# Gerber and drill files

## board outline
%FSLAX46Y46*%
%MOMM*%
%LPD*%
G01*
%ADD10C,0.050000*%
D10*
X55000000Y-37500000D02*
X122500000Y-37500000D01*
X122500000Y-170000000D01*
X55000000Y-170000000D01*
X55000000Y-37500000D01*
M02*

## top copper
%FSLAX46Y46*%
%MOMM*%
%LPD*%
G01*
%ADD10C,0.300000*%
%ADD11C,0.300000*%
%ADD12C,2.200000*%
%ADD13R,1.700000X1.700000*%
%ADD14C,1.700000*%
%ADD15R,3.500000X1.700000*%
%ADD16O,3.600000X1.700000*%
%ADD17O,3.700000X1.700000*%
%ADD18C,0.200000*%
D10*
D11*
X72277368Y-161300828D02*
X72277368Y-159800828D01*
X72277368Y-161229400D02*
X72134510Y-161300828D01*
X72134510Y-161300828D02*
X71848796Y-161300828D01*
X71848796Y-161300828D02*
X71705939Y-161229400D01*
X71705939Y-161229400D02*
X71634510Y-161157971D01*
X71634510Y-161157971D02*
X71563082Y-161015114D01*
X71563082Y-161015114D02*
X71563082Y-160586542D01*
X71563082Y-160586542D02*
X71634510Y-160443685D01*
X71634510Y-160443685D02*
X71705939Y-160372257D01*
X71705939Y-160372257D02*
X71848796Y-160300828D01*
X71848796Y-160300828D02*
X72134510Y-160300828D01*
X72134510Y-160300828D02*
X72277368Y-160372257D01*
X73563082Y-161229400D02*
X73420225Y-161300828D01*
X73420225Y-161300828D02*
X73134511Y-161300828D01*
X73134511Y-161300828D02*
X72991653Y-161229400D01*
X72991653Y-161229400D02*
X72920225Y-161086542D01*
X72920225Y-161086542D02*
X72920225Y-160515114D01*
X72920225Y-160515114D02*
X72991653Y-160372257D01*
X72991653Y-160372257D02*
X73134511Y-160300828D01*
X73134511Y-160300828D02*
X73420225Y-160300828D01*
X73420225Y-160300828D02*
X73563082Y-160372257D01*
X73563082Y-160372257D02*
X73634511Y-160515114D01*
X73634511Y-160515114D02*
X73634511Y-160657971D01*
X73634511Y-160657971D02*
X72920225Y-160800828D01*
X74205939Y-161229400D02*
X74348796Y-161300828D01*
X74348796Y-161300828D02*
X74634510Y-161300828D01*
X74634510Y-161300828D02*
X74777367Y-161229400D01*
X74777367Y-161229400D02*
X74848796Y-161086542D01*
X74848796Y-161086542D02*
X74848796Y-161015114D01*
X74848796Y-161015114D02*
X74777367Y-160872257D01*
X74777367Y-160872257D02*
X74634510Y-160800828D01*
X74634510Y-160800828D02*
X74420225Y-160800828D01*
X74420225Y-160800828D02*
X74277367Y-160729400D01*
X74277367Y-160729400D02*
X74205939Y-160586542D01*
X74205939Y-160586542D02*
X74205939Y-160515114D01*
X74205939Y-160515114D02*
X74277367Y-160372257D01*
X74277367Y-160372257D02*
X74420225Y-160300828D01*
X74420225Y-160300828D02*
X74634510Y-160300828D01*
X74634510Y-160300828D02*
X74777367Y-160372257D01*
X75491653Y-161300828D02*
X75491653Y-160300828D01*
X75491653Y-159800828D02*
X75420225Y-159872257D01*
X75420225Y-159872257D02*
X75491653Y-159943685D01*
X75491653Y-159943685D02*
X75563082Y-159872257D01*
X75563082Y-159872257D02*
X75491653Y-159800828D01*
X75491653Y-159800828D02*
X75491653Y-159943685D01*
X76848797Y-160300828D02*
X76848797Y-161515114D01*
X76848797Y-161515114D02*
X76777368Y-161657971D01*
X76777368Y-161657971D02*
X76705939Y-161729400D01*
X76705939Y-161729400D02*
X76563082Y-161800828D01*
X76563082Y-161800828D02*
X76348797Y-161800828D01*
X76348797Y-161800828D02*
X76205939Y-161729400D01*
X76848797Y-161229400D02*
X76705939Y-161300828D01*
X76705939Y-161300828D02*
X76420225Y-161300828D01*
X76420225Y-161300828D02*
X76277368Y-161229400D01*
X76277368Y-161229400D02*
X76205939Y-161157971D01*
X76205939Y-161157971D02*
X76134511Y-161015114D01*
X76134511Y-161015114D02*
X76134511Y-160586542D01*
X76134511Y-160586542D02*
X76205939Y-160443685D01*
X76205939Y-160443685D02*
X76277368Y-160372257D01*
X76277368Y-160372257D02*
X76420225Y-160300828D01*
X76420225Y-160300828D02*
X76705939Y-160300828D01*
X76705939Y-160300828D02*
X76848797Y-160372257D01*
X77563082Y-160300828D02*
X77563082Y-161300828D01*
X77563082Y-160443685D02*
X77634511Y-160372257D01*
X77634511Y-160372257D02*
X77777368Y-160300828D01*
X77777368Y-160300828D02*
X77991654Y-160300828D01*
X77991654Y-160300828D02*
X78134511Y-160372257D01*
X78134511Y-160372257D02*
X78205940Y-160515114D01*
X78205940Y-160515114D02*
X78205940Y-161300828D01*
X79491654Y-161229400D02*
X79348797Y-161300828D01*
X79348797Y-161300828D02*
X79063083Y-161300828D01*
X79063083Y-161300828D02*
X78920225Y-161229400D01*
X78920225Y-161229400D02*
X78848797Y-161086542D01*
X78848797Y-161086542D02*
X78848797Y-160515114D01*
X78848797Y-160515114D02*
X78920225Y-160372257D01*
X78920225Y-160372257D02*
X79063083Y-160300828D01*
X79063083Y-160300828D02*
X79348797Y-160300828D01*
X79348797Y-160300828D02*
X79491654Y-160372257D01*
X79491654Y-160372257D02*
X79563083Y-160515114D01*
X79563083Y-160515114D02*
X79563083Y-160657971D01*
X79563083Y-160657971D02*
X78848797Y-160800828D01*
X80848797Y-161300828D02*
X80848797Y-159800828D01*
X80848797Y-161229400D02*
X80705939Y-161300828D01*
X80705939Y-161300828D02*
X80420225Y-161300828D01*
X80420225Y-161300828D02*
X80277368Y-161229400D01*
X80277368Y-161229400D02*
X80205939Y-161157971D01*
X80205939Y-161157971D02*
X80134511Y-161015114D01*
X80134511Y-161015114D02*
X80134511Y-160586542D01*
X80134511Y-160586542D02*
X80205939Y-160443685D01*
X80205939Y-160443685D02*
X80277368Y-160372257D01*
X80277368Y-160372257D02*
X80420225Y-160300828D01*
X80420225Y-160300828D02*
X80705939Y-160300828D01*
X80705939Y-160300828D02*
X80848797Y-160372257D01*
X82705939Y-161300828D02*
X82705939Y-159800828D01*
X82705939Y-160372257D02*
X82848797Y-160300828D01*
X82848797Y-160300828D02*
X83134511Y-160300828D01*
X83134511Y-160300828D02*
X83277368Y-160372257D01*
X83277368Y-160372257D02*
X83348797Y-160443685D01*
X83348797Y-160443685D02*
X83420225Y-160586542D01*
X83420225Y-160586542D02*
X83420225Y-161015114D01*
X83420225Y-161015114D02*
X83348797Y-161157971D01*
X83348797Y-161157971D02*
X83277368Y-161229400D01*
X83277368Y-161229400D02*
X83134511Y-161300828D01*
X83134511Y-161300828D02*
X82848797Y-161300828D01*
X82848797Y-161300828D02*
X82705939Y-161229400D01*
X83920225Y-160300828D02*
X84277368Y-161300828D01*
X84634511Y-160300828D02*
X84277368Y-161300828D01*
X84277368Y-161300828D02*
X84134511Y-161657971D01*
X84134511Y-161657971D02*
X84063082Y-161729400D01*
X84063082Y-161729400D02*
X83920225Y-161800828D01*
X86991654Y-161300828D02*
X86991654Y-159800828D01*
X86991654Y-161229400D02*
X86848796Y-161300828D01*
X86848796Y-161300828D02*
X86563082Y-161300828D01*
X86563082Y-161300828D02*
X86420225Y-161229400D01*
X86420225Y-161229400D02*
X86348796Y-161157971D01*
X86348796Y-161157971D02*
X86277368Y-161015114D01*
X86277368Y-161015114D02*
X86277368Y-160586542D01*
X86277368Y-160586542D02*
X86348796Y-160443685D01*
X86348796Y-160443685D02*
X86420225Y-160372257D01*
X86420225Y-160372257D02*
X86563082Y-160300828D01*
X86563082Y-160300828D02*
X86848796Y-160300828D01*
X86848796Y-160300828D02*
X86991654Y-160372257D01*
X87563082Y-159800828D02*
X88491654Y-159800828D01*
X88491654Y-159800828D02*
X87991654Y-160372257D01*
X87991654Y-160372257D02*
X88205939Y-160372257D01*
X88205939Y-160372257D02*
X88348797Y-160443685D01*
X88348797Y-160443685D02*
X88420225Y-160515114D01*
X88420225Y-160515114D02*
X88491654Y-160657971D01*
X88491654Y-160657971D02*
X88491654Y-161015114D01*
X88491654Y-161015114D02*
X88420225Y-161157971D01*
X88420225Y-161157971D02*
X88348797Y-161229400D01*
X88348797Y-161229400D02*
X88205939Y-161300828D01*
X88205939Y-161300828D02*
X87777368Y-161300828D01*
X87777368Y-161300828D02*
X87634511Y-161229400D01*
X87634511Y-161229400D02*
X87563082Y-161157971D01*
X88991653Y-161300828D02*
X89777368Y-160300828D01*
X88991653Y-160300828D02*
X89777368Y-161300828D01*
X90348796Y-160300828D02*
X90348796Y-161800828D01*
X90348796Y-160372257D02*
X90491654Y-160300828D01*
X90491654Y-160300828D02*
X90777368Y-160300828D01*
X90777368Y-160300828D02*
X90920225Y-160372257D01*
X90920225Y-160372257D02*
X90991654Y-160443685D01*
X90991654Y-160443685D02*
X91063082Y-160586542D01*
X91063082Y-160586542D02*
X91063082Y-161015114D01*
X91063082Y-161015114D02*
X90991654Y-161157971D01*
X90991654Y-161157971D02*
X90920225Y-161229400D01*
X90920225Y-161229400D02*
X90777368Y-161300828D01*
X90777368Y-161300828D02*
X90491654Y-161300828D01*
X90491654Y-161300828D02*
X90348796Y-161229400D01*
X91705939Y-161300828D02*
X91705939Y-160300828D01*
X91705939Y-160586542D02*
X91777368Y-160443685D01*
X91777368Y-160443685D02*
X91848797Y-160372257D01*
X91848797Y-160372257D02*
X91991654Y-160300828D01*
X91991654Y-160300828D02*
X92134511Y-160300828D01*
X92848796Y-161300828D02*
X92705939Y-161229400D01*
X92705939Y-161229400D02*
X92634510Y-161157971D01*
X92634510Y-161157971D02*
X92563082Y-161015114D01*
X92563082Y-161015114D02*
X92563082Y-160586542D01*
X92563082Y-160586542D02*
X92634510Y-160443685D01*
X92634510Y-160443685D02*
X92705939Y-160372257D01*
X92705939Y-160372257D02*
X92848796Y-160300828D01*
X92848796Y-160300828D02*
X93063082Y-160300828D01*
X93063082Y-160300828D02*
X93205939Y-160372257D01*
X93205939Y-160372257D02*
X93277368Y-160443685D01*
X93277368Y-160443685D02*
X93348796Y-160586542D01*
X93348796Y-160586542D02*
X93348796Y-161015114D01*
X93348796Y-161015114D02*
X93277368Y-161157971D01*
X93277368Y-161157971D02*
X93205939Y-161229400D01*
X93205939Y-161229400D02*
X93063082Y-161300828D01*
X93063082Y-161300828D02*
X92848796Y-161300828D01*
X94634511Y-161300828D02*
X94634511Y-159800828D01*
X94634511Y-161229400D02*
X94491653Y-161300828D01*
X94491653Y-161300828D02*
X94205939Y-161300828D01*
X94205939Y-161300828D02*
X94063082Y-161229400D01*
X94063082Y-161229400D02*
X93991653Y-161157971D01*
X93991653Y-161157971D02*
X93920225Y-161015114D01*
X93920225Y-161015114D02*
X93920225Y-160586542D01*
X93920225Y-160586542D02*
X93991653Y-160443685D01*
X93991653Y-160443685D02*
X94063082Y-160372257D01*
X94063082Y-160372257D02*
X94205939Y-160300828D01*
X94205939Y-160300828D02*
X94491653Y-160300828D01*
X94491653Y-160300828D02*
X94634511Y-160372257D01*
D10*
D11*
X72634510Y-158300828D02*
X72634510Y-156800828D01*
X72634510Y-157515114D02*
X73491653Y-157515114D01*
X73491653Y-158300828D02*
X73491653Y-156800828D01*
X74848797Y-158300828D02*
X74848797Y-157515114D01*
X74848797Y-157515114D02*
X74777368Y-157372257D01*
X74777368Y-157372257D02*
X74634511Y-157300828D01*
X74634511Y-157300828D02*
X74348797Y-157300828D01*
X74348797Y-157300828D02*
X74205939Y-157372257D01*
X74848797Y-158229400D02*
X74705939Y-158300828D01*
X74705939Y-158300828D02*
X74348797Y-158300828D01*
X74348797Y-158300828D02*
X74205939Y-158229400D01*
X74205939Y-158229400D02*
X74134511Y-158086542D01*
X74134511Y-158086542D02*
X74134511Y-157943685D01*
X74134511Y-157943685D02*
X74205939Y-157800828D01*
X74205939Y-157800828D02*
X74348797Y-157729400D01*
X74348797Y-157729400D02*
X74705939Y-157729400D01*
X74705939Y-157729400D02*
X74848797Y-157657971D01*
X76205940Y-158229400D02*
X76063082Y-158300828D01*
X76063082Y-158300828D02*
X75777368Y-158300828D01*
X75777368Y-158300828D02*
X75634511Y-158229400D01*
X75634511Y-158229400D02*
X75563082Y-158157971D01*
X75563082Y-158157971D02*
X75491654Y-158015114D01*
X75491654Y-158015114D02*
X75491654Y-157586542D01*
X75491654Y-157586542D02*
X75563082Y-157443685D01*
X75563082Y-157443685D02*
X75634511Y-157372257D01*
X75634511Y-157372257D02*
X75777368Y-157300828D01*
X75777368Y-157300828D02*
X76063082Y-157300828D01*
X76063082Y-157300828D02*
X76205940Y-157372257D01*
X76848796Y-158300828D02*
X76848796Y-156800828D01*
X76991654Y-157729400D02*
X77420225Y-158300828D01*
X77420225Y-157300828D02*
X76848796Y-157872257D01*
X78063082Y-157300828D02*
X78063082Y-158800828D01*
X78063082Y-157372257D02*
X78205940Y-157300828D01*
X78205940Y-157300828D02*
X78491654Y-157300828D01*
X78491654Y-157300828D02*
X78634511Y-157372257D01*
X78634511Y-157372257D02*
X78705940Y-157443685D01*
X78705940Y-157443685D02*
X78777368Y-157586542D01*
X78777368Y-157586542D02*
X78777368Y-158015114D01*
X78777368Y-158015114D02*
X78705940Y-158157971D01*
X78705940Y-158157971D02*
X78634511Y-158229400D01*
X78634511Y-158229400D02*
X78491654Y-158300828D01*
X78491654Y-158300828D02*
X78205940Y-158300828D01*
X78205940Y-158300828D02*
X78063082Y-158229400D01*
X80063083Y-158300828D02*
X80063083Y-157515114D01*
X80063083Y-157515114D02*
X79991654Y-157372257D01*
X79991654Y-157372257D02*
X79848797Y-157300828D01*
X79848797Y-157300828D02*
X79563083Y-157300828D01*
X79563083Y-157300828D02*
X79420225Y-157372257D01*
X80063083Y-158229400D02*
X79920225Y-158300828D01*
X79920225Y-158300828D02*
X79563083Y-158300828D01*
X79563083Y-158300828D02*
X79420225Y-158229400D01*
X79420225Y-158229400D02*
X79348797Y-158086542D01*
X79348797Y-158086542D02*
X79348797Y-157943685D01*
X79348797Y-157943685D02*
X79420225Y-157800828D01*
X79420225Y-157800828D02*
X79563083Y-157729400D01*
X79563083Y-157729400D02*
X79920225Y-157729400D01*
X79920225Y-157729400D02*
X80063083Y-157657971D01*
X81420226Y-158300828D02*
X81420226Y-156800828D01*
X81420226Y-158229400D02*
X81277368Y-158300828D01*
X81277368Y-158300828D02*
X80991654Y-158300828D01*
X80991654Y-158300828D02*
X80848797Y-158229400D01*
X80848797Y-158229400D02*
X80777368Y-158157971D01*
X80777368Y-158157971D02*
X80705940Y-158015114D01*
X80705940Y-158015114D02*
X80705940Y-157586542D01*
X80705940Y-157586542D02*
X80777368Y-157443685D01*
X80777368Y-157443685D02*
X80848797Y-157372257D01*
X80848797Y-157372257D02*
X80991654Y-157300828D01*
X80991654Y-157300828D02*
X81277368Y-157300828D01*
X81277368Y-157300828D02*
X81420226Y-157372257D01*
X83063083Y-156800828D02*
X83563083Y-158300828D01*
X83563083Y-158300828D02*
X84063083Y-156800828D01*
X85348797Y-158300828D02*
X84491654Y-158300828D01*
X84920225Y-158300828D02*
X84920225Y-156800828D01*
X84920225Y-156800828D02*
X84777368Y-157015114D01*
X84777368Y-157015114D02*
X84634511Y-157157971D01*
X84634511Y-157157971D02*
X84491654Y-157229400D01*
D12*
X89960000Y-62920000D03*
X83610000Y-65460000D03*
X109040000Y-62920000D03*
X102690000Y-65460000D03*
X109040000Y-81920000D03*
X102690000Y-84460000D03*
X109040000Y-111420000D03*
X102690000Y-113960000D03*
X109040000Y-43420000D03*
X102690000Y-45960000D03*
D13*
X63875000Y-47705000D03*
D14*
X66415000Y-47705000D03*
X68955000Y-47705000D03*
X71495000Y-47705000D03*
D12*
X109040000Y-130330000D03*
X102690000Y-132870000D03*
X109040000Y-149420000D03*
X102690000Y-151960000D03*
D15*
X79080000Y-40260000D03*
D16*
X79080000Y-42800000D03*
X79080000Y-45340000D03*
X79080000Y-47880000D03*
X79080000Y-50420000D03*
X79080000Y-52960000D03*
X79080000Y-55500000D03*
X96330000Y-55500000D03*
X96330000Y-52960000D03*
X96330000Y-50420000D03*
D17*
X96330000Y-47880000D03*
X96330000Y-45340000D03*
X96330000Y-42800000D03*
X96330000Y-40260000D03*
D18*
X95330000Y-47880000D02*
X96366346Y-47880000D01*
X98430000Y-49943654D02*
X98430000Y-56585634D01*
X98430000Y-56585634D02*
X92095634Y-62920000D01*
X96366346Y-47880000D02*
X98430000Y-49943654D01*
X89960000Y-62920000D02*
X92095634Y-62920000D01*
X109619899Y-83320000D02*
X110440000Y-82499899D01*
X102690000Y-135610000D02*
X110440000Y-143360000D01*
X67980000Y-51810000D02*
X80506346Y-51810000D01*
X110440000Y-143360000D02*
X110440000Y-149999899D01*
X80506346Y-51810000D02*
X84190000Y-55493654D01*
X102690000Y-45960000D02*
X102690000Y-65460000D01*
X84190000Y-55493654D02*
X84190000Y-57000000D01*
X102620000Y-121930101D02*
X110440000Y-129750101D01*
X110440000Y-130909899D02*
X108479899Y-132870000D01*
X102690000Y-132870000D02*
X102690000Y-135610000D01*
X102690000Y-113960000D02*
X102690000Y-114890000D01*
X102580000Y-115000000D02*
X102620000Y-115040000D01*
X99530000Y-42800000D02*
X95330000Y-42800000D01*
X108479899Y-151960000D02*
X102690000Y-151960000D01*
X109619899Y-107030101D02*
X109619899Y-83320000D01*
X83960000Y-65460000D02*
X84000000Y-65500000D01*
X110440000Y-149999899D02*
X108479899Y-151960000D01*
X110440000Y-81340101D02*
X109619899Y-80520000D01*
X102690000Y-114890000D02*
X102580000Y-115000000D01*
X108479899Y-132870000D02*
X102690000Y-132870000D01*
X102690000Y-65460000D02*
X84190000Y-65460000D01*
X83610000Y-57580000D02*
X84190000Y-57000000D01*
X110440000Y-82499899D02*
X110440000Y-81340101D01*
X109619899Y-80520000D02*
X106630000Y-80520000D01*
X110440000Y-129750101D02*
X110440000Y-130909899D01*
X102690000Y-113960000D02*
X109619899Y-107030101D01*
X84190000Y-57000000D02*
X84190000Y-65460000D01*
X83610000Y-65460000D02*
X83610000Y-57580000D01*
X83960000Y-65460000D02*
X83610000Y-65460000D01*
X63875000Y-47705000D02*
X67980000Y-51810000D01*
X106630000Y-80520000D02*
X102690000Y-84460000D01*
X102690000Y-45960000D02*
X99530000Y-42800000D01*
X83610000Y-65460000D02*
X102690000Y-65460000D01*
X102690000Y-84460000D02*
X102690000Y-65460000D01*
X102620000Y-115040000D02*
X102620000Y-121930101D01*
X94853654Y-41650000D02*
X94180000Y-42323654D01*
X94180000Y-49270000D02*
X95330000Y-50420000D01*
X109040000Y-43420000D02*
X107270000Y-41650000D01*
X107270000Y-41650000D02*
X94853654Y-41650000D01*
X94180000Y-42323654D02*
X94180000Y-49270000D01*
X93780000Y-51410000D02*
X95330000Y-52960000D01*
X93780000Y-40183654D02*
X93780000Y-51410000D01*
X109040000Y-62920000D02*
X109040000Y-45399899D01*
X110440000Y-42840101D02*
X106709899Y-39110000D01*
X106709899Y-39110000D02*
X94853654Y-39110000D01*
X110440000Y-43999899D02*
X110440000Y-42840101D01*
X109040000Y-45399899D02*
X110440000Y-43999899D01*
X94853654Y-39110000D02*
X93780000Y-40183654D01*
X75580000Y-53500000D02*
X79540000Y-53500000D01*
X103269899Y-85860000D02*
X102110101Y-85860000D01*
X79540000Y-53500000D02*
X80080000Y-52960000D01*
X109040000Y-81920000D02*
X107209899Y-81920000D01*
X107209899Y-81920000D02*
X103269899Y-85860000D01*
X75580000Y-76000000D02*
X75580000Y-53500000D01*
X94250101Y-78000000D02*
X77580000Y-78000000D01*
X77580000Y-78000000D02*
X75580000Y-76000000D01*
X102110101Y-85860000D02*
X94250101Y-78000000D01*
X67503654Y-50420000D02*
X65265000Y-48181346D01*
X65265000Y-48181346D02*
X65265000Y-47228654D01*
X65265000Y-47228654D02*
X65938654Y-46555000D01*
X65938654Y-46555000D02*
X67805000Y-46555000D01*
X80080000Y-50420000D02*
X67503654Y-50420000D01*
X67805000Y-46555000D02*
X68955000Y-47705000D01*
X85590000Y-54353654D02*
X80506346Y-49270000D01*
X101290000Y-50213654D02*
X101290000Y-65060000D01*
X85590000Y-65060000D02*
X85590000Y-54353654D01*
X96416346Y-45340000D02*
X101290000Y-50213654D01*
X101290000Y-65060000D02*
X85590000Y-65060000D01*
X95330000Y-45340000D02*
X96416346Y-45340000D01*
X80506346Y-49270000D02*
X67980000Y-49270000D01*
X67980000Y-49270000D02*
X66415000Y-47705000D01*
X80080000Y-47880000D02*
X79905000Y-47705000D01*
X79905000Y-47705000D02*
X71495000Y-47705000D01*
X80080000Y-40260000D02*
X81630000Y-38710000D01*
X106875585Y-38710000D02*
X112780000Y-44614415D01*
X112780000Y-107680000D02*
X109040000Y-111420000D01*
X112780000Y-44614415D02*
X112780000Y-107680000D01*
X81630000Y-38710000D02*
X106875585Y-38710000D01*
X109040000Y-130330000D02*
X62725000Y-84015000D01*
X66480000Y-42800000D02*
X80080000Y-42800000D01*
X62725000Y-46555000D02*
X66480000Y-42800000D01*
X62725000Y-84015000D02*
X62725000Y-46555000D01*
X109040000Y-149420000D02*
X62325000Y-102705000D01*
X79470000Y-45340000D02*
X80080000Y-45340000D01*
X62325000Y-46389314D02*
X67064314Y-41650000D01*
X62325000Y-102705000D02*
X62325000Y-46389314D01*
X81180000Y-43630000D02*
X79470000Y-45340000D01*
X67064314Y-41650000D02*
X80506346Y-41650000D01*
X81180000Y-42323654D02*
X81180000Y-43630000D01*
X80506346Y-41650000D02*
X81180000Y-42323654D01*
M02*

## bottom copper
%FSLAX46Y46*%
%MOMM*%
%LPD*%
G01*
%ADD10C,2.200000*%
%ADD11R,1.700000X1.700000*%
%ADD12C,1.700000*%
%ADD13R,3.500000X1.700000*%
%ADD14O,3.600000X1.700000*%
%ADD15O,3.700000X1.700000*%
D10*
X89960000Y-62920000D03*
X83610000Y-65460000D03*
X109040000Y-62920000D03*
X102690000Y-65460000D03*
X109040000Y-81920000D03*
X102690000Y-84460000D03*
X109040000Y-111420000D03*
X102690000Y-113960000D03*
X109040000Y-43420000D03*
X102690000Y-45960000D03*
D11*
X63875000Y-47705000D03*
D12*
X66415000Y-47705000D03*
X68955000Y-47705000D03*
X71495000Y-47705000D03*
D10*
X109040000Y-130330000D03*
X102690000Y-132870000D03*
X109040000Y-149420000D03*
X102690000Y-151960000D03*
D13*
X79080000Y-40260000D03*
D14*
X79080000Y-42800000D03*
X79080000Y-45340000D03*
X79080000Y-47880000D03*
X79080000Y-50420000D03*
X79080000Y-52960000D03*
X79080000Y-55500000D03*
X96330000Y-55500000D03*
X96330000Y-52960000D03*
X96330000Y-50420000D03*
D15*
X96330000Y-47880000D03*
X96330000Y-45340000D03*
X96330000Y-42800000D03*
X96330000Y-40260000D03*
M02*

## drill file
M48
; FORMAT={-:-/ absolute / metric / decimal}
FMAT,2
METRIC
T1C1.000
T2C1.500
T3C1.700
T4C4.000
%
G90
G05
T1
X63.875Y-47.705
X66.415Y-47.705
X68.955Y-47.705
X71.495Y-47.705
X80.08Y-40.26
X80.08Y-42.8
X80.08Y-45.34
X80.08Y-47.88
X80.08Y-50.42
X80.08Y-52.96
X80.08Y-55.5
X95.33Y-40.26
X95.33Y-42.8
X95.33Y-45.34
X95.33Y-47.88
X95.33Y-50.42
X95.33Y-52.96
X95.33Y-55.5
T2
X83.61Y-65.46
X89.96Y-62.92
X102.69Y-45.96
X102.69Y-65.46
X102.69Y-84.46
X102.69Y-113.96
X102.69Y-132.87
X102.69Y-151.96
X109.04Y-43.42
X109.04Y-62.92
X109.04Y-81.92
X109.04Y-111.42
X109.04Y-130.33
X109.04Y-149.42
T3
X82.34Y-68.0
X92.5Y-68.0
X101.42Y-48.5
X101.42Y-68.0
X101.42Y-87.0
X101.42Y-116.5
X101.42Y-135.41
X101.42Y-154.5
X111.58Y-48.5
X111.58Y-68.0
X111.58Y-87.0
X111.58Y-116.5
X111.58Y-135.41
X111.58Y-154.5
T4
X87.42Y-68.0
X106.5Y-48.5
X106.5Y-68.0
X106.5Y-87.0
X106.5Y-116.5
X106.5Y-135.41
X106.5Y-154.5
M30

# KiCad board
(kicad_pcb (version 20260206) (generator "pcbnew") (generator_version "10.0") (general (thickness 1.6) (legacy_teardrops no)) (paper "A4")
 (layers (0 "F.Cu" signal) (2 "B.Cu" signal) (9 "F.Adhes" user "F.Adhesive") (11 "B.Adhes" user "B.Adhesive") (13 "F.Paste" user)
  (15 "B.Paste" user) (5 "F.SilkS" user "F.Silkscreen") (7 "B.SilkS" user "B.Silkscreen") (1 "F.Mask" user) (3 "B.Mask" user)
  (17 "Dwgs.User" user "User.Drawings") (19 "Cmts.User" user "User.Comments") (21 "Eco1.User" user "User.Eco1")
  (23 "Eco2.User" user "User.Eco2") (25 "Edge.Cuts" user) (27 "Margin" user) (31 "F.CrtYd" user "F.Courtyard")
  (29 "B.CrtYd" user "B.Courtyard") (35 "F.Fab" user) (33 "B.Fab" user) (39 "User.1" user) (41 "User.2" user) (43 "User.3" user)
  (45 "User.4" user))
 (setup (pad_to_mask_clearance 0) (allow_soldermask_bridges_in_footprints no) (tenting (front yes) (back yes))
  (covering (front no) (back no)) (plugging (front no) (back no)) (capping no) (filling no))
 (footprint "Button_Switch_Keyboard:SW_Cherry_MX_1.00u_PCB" (layer "F.Cu") (at 89.96 62.92)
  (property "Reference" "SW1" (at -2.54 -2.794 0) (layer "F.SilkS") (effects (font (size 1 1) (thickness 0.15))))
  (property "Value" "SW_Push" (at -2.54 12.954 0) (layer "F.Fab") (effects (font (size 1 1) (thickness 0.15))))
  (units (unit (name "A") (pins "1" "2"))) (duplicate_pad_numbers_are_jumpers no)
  (pad "" np_thru_hole circle (at -7.62 5.08) (size 1.7 1.7) (drill 1.7) (layers "*.Cu" "*.Mask"))
  (pad "" np_thru_hole circle (at -2.54 5.08) (size 4 4) (drill 4) (layers "*.Cu" "*.Mask"))
  (pad "" np_thru_hole circle (at 2.54 5.08) (size 1.7 1.7) (drill 1.7) (layers "*.Cu" "*.Mask"))
  (pad "1" thru_hole circle (at 0 0) (size 2.2 2.2) (drill 1.5) (layers "*.Cu" "*.Mask") (remove_unused_layers no)
   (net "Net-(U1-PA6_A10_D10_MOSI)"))
  (pad "2" thru_hole circle (at -6.35 2.54) (size 2.2 2.2) (drill 1.5) (layers "*.Cu" "*.Mask") (remove_unused_layers no) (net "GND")))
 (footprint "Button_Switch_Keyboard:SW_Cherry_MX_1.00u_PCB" (layer "F.Cu") (at 109.04 62.92)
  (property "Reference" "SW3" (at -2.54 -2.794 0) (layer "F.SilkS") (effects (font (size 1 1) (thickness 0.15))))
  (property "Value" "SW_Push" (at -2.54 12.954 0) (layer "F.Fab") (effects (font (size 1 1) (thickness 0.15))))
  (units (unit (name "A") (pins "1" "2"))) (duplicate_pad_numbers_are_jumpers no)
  (pad "" np_thru_hole circle (at -7.62 5.08) (size 1.7 1.7) (drill 1.7) (layers "*.Cu" "*.Mask"))
  (pad "" np_thru_hole circle (at -2.54 5.08) (size 4 4) (drill 4) (layers "*.Cu" "*.Mask"))
  (pad "" np_thru_hole circle (at 2.54 5.08) (size 1.7 1.7) (drill 1.7) (layers "*.Cu" "*.Mask"))
  (pad "1" thru_hole circle (at 0 0) (size 2.2 2.2) (drill 1.5) (layers "*.Cu" "*.Mask") (remove_unused_layers no)
   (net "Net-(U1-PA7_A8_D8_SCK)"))
  (pad "2" thru_hole circle (at -6.35 2.54) (size 2.2 2.2) (drill 1.5) (layers "*.Cu" "*.Mask") (remove_unused_layers no) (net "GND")))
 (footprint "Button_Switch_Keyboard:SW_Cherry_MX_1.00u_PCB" (layer "F.Cu") (at 109.04 81.92)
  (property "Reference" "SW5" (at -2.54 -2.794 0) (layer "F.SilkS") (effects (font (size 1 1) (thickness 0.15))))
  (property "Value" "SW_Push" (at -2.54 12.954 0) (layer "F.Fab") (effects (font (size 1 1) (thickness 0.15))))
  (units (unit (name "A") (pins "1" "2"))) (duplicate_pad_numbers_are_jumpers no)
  (pad "" np_thru_hole circle (at -7.62 5.08) (size 1.7 1.7) (drill 1.7) (layers "*.Cu" "*.Mask"))
  (pad "" np_thru_hole circle (at -2.54 5.08) (size 4 4) (drill 4) (layers "*.Cu" "*.Mask"))
  (pad "" np_thru_hole circle (at 2.54 5.08) (size 1.7 1.7) (drill 1.7) (layers "*.Cu" "*.Mask"))
  (pad "1" thru_hole circle (at 0 0) (size 2.2 2.2) (drill 1.5) (layers "*.Cu" "*.Mask") (remove_unused_layers no)
   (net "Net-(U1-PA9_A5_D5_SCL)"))
  (pad "2" thru_hole circle (at -6.35 2.54) (size 2.2 2.2) (drill 1.5) (layers "*.Cu" "*.Mask") (remove_unused_layers no) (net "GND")))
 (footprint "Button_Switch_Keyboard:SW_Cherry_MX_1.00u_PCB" (layer "F.Cu") (at 109.04 111.42)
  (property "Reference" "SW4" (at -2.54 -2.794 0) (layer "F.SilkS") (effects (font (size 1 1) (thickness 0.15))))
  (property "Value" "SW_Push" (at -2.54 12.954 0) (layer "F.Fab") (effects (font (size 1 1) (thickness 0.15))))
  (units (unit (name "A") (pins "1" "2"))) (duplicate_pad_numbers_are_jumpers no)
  (pad "" np_thru_hole circle (at -7.62 5.08) (size 1.7 1.7) (drill 1.7) (layers "*.Cu" "*.Mask"))
  (pad "" np_thru_hole circle (at -2.54 5.08) (size 4 4) (drill 4) (layers "*.Cu" "*.Mask"))
  (pad "" np_thru_hole circle (at 2.54 5.08) (size 1.7 1.7) (drill 1.7) (layers "*.Cu" "*.Mask"))
  (pad "1" thru_hole circle (at 0 0) (size 2.2 2.2) (drill 1.5) (layers "*.Cu" "*.Mask") (remove_unused_layers no)
   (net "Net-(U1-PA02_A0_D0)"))
  (pad "2" thru_hole circle (at -6.35 2.54) (size 2.2 2.2) (drill 1.5) (layers "*.Cu" "*.Mask") (remove_unused_layers no) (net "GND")))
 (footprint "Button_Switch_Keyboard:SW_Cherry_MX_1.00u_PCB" (layer "F.Cu") (at 109.04 43.42)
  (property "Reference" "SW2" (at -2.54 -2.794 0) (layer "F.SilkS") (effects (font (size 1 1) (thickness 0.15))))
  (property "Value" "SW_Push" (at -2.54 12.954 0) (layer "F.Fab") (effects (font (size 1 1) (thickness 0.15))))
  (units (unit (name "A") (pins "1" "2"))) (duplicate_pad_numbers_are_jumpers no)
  (pad "" np_thru_hole circle (at -7.62 5.08) (size 1.7 1.7) (drill 1.7) (layers "*.Cu" "*.Mask"))
  (pad "" np_thru_hole circle (at -2.54 5.08) (size 4 4) (drill 4) (layers "*.Cu" "*.Mask"))
  (pad "" np_thru_hole circle (at 2.54 5.08) (size 1.7 1.7) (drill 1.7) (layers "*.Cu" "*.Mask"))
  (pad "1" thru_hole circle (at 0 0) (size 2.2 2.2) (drill 1.5) (layers "*.Cu" "*.Mask") (remove_unused_layers no)
   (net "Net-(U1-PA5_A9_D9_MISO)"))
  (pad "2" thru_hole circle (at -6.35 2.54) (size 2.2 2.2) (drill 1.5) (layers "*.Cu" "*.Mask") (remove_unused_layers no) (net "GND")))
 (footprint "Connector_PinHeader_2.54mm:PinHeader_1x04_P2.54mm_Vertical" (layer "F.Cu") (at 63.875 47.705 90)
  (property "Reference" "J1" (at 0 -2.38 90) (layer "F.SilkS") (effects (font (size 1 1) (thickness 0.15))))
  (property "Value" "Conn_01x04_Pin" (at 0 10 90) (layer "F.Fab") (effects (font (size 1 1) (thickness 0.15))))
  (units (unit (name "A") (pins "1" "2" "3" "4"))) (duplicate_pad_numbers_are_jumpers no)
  (pad "1" thru_hole rect (at 0 0 90) (size 1.7 1.7) (drill 1) (layers "*.Cu" "*.Mask") (remove_unused_layers no) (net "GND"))
  (pad "2" thru_hole circle (at 0 2.54 90) (size 1.7 1.7) (drill 1) (layers "*.Cu" "*.Mask") (remove_unused_layers no)
   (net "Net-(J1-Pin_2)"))
  (pad "3" thru_hole circle (at 0 5.08 90) (size 1.7 1.7) (drill 1) (layers "*.Cu" "*.Mask") (remove_unused_layers no)
   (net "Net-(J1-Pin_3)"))
  (pad "4" thru_hole circle (at 0 7.62 90) (size 1.7 1.7) (drill 1) (layers "*.Cu" "*.Mask") (remove_unused_layers no)
   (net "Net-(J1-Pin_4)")))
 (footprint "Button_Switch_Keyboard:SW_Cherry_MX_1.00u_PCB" (layer "F.Cu") (at 109.04 130.33)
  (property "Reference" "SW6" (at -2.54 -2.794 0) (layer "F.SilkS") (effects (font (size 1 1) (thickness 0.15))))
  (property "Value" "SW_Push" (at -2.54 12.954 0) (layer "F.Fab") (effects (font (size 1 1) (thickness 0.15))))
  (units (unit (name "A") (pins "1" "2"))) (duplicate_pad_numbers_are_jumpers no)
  (pad "" np_thru_hole circle (at -7.62 5.08) (size 1.7 1.7) (drill 1.7) (layers "*.Cu" "*.Mask"))
  (pad "" np_thru_hole circle (at -2.54 5.08) (size 4 4) (drill 4) (layers "*.Cu" "*.Mask"))
  (pad "" np_thru_hole circle (at 2.54 5.08) (size 1.7 1.7) (drill 1.7) (layers "*.Cu" "*.Mask"))
  (pad "1" thru_hole circle (at 0 0) (size 2.2 2.2) (drill 1.5) (layers "*.Cu" "*.Mask") (remove_unused_layers no)
   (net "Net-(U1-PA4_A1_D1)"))
  (pad "2" thru_hole circle (at -6.35 2.54) (size 2.2 2.2) (drill 1.5) (layers "*.Cu" "*.Mask") (remove_unused_layers no) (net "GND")))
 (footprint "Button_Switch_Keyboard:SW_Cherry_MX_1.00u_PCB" (layer "F.Cu") (at 109.04 149.42)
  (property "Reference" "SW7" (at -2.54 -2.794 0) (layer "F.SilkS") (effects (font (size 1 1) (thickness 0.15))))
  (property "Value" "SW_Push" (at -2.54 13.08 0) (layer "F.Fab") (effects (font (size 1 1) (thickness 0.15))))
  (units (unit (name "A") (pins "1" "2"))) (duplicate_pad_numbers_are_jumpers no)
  (pad "" np_thru_hole circle (at -7.62 5.08) (size 1.7 1.7) (drill 1.7) (layers "*.Cu" "*.Mask"))
  (pad "" np_thru_hole circle (at -2.54 5.08) (size 4 4) (drill 4) (layers "*.Cu" "*.Mask"))
  (pad "" np_thru_hole circle (at 2.54 5.08) (size 1.7 1.7) (drill 1.7) (layers "*.Cu" "*.Mask"))
  (pad "1" thru_hole circle (at 0 0) (size 2.2 2.2) (drill 1.5) (layers "*.Cu" "*.Mask") (remove_unused_layers no)
   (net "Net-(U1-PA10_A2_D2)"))
  (pad "2" thru_hole circle (at -6.35 2.54) (size 2.2 2.2) (drill 1.5) (layers "*.Cu" "*.Mask") (remove_unused_layers no) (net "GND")))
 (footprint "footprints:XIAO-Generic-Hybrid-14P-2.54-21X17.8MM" (layer "F.Cu") (at 87.705 47.88)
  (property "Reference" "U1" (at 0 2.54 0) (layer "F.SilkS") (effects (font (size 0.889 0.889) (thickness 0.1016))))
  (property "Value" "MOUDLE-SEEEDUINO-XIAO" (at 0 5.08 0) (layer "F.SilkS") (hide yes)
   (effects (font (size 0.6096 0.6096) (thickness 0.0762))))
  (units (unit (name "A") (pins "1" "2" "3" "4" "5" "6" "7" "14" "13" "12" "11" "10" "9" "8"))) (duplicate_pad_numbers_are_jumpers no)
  (pad "1" thru_hole rect (at -7.625 -7.62) (size 3.5 1.7) (drill 1 (offset -1 0)) (layers "*.Cu" "*.Mask") (remove_unused_layers no)
   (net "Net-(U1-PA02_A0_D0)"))
  (pad "2" thru_hole oval (at -7.625 -5.08) (size 3.6 1.7) (drill 1 (offset -1 0)) (layers "*.Cu" "*.Mask") (remove_unused_layers no)
   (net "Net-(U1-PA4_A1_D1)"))
  (pad "3" thru_hole oval (at -7.625 -2.54) (size 3.6 1.7) (drill 1 (offset -1 0)) (layers "*.Cu" "*.Mask") (remove_unused_layers no)
   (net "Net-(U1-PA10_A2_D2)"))
  (pad "4" thru_hole oval (at -7.625 0) (size 3.6 1.7) (drill 1 (offset -1 0)) (layers "*.Cu" "*.Mask") (remove_unused_layers no)
   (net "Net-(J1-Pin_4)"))
  (pad "5" thru_hole oval (at -7.625 2.54) (size 3.6 1.7) (drill 1 (offset -1 0)) (layers "*.Cu" "*.Mask") (remove_unused_layers no)
   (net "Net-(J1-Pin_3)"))
  (pad "6" thru_hole oval (at -7.625 5.08 180) (size 3.6 1.7) (drill 1 (offset 1 0)) (layers "*.Cu" "*.Mask") (remove_unused_layers no)
   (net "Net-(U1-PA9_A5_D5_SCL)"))
  (pad "7" thru_hole oval (at -7.625 7.62) (size 3.6 1.7) (drill 1 (offset -1 0)) (layers "*.Cu" "*.Mask") (remove_unused_layers no)
   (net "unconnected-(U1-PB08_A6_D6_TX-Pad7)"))
  (pad "8" thru_hole oval (at 7.625 7.62) (size 3.6 1.7) (drill 1 (offset 1 0)) (layers "*.Cu" "*.Mask") (remove_unused_layers no)
   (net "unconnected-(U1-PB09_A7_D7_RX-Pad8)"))
  (pad "9" thru_hole oval (at 7.625 5.08) (size 3.6 1.7) (drill 1 (offset 1 0)) (layers "*.Cu" "*.Mask") (remove_unused_layers no)
   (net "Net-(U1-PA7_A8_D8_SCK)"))
  (pad "10" thru_hole oval (at 7.625 2.54) (size 3.6 1.7) (drill 1 (offset 1 0)) (layers "*.Cu" "*.Mask") (remove_unused_layers no)
   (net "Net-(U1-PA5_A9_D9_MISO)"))
  (pad "11" thru_hole oval (at 7.625 0) (size 3.7 1.7) (drill 1 (offset 1 0)) (layers "*.Cu" "*.Mask") (remove_unused_layers no)
   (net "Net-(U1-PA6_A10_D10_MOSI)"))
  (pad "12" thru_hole oval (at 7.625 -2.54) (size 3.7 1.7) (drill 1 (offset 1 0)) (layers "*.Cu" "*.Mask") (remove_unused_layers no)
   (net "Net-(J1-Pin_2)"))
  (pad "13" thru_hole oval (at 7.625 -5.08) (size 3.7 1.7) (drill 1 (offset 1 0)) (layers "*.Cu" "*.Mask") (remove_unused_layers no)
   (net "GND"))
  (pad "14" thru_hole oval (at 7.625 -7.62) (size 3.7 1.7) (drill 1 (offset 1 0)) (layers "*.Cu" "*.Mask") (remove_unused_layers no)
   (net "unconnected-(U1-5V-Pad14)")))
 (gr_rect (start 55 37.5) (end 122.5 170) (stroke (width 0.05) (type default)) (fill no) (layer "Edge.Cuts"))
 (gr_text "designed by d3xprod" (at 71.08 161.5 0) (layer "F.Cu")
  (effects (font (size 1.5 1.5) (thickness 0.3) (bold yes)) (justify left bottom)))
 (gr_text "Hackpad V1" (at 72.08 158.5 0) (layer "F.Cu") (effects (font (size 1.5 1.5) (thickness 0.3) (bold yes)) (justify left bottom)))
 (segment (start 95.33 47.88) (end 96.366346 47.88) (width 0.2) (layer "F.Cu") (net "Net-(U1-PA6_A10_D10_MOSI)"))
 (segment (start 98.43 49.943654) (end 98.43 56.585634) (width 0.2) (layer "F.Cu") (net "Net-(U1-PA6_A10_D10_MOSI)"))
 (segment (start 98.43 56.585634) (end 92.095634 62.92) (width 0.2) (layer "F.Cu") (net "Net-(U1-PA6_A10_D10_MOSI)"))
 (segment (start 96.366346 47.88) (end 98.43 49.943654) (width 0.2) (layer "F.Cu") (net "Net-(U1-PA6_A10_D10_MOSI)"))
 (segment (start 89.96 62.92) (end 92.095634 62.92) (width 0.2) (layer "F.Cu") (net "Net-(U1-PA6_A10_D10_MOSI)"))
 (segment (start 109.619899 83.32) (end 110.44 82.499899) (width 0.2) (layer "F.Cu") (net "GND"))
 (segment (start 102.69 135.61) (end 110.44 143.36) (width 0.2) (layer "F.Cu") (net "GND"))
 (segment (start 67.98 51.81) (end 80.506346 51.81) (width 0.2) (layer "F.Cu") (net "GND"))
 (segment (start 110.44 143.36) (end 110.44 149.999899) (width 0.2) (layer "F.Cu") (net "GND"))
 (segment (start 80.506346 51.81) (end 84.19 55.493654) (width 0.2) (layer "F.Cu") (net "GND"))
 (segment (start 102.69 45.96) (end 102.69 65.46) (width 0.2) (layer "F.Cu") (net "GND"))
 (segment (start 84.19 55.493654) (end 84.19 57) (width 0.2) (layer "F.Cu") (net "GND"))
 (segment (start 102.62 121.930101) (end 110.44 129.750101) (width 0.2) (layer "F.Cu") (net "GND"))
 (segment (start 110.44 130.909899) (end 108.479899 132.87) (width 0.2) (layer "F.Cu") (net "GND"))
 (segment (start 102.69 132.87) (end 102.69 135.61) (width 0.2) (layer "F.Cu") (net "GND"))
 (segment (start 102.69 113.96) (end 102.69 114.89) (width 0.2) (layer "F.Cu") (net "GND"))
 (segment (start 102.58 115) (end 102.62 115.04) (width 0.2) (layer "F.Cu") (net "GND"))
 (segment (start 99.53 42.8) (end 95.33 42.8) (width 0.2) (layer "F.Cu") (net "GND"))
 (segment (start 108.479899 151.96) (end 102.69 151.96) (width 0.2) (layer "F.Cu") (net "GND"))
 (segment (start 109.619899 107.030101) (end 109.619899 83.32) (width 0.2) (layer "F.Cu") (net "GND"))
 (segment (start 83.96 65.46) (end 84 65.5) (width 0.2) (layer "F.Cu") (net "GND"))
 (segment (start 110.44 149.999899) (end 108.479899 151.96) (width 0.2) (layer "F.Cu") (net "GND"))
 (segment (start 110.44 81.340101) (end 109.619899 80.52) (width 0.2) (layer "F.Cu") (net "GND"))
 (segment (start 102.69 114.89) (end 102.58 115) (width 0.2) (layer "F.Cu") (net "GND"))
 (segment (start 108.479899 132.87) (end 102.69 132.87) (width 0.2) (layer "F.Cu") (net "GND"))
 (segment (start 102.69 65.46) (end 84.19 65.46) (width 0.2) (layer "F.Cu") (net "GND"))
 (segment (start 83.61 57.58) (end 84.19 57) (width 0.2) (layer "F.Cu") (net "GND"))
 (segment (start 110.44 82.499899) (end 110.44 81.340101) (width 0.2) (layer "F.Cu") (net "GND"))
 (segment (start 109.619899 80.52) (end 106.63 80.52) (width 0.2) (layer "F.Cu") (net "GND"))
 (segment (start 110.44 129.750101) (end 110.44 130.909899) (width 0.2) (layer "F.Cu") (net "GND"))
 (segment (start 102.69 113.96) (end 109.619899 107.030101) (width 0.2) (layer "F.Cu") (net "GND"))
 (segment (start 84.19 57) (end 84.19 65.46) (width 0.2) (layer "F.Cu") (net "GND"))
 (segment (start 83.61 65.46) (end 83.61 57.58) (width 0.2) (layer "F.Cu") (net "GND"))
 (segment (start 83.96 65.46) (end 83.61 65.46) (width 0.2) (layer "F.Cu") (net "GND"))
 (segment (start 63.875 47.705) (end 67.98 51.81) (width 0.2) (layer "F.Cu") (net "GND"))
 (segment (start 106.63 80.52) (end 102.69 84.46) (width 0.2) (layer "F.Cu") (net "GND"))
 (segment (start 102.69 45.96) (end 99.53 42.8) (width 0.2) (layer "F.Cu") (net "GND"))
 (segment (start 83.61 65.46) (end 102.69 65.46) (width 0.2) (layer "F.Cu") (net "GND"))
 (segment (start 102.69 84.46) (end 102.69 65.46) (width 0.2) (layer "F.Cu") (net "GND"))
 (segment (start 102.62 115.04) (end 102.62 121.930101) (width 0.2) (layer "F.Cu") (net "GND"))
 (segment (start 94.853654 41.65) (end 94.18 42.323654) (width 0.2) (layer "F.Cu") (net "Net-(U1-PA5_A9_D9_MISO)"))
 (segment (start 94.18 49.27) (end 95.33 50.42) (width 0.2) (layer "F.Cu") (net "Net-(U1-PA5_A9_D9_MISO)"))
 (segment (start 109.04 43.42) (end 107.27 41.65) (width 0.2) (layer "F.Cu") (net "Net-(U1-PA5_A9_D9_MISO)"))
 (segment (start 107.27 41.65) (end 94.853654 41.65) (width 0.2) (layer "F.Cu") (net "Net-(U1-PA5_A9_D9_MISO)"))
 (segment (start 94.18 42.323654) (end 94.18 49.27) (width 0.2) (layer "F.Cu") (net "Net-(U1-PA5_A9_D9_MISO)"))
 (segment (start 93.78 51.41) (end 95.33 52.96) (width 0.2) (layer "F.Cu") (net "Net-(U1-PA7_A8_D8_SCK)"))
 (segment (start 93.78 40.183654) (end 93.78 51.41) (width 0.2) (layer "F.Cu") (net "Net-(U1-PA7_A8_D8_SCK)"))
 (segment (start 109.04 62.92) (end 109.04 45.399899) (width 0.2) (layer "F.Cu") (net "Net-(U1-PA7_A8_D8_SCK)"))
 (segment (start 110.44 42.840101) (end 106.709899 39.11) (width 0.2) (layer "F.Cu") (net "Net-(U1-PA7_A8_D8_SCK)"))
 (segment (start 106.709899 39.11) (end 94.853654 39.11) (width 0.2) (layer "F.Cu") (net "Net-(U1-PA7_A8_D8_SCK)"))
 (segment (start 110.44 43.999899) (end 110.44 42.840101) (width 0.2) (layer "F.Cu") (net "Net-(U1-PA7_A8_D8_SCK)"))
 (segment (start 109.04 45.399899) (end 110.44 43.999899) (width 0.2) (layer "F.Cu") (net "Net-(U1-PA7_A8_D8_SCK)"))
 (segment (start 94.853654 39.11) (end 93.78 40.183654) (width 0.2) (layer "F.Cu") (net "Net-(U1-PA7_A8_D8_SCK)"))
 (segment (start 75.58 53.5) (end 79.54 53.5) (width 0.2) (layer "F.Cu") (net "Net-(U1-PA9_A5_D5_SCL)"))
 (segment (start 103.269899 85.86) (end 102.110101 85.86) (width 0.2) (layer "F.Cu") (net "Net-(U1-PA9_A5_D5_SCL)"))
 (segment (start 79.54 53.5) (end 80.08 52.96) (width 0.2) (layer "F.Cu") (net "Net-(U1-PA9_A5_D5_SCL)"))
 (segment (start 109.04 81.92) (end 107.209899 81.92) (width 0.2) (layer "F.Cu") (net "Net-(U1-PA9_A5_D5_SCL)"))
 (segment (start 107.209899 81.92) (end 103.269899 85.86) (width 0.2) (layer "F.Cu") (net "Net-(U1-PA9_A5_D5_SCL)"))
 (segment (start 75.58 76) (end 75.58 53.5) (width 0.2) (layer "F.Cu") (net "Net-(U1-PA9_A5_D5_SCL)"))
 (segment (start 94.250101 78) (end 77.58 78) (width 0.2) (layer "F.Cu") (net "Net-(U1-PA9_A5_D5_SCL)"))
 (segment (start 77.58 78) (end 75.58 76) (width 0.2) (layer "F.Cu") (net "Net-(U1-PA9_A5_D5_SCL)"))
 (segment (start 102.110101 85.86) (end 94.250101 78) (width 0.2) (layer "F.Cu") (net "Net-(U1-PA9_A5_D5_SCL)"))
 (segment (start 67.503654 50.42) (end 65.265 48.181346) (width 0.2) (layer "F.Cu") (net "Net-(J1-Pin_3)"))
 (segment (start 65.265 48.181346) (end 65.265 47.228654) (width 0.2) (layer "F.Cu") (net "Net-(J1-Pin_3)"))
 (segment (start 65.265 47.228654) (end 65.938654 46.555) (width 0.2) (layer "F.Cu") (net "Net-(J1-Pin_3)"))
 (segment (start 65.938654 46.555) (end 67.805 46.555) (width 0.2) (layer "F.Cu") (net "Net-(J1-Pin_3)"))
 (segment (start 80.08 50.42) (end 67.503654 50.42) (width 0.2) (layer "F.Cu") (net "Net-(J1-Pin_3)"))
 (segment (start 67.805 46.555) (end 68.955 47.705) (width 0.2) (layer "F.Cu") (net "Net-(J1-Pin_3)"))
 (segment (start 85.59 54.353654) (end 80.506346 49.27) (width 0.2) (layer "F.Cu") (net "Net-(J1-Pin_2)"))
 (segment (start 101.29 50.213654) (end 101.29 65.06) (width 0.2) (layer "F.Cu") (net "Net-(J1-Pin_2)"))
 (segment (start 85.59 65.06) (end 85.59 54.353654) (width 0.2) (layer "F.Cu") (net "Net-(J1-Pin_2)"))
 (segment (start 96.416346 45.34) (end 101.29 50.213654) (width 0.2) (layer "F.Cu") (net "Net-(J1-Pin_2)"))
 (segment (start 101.29 65.06) (end 85.59 65.06) (width 0.2) (layer "F.Cu") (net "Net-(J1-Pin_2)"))
 (segment (start 95.33 45.34) (end 96.416346 45.34) (width 0.2) (layer "F.Cu") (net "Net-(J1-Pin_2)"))
 (segment (start 80.506346 49.27) (end 67.98 49.27) (width 0.2) (layer "F.Cu") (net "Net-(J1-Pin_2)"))
 (segment (start 67.98 49.27) (end 66.415 47.705) (width 0.2) (layer "F.Cu") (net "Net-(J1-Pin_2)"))
 (segment (start 80.08 47.88) (end 79.905 47.705) (width 0.2) (layer "F.Cu") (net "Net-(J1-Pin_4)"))
 (segment (start 79.905 47.705) (end 71.495 47.705) (width 0.2) (layer "F.Cu") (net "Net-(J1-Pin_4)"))
 (segment (start 80.08 40.26) (end 81.63 38.71) (width 0.2) (layer "F.Cu") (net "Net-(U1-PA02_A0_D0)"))
 (segment (start 106.875585 38.71) (end 112.78 44.614415) (width 0.2) (layer "F.Cu") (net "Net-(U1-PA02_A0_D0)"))
 (segment (start 112.78 107.68) (end 109.04 111.42) (width 0.2) (layer "F.Cu") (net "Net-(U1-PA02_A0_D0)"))
 (segment (start 112.78 44.614415) (end 112.78 107.68) (width 0.2) (layer "F.Cu") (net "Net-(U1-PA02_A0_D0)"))
 (segment (start 81.63 38.71) (end 106.875585 38.71) (width 0.2) (layer "F.Cu") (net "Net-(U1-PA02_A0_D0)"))
 (segment (start 109.04 130.33) (end 62.725 84.015) (width 0.2) (layer "F.Cu") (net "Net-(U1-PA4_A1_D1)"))
 (segment (start 66.48 42.8) (end 80.08 42.8) (width 0.2) (layer "F.Cu") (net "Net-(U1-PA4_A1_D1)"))
 (segment (start 62.725 46.555) (end 66.48 42.8) (width 0.2) (layer "F.Cu") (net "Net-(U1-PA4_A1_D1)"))
 (segment (start 62.725 84.015) (end 62.725 46.555) (width 0.2) (layer "F.Cu") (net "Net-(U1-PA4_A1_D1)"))
 (segment (start 109.04 149.42) (end 62.325 102.705) (width 0.2) (layer "F.Cu") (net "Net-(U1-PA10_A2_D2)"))
 (segment (start 79.47 45.34) (end 80.08 45.34) (width 0.2) (layer "F.Cu") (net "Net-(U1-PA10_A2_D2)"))
 (segment (start 62.325 46.389314) (end 67.064314 41.65) (width 0.2) (layer "F.Cu") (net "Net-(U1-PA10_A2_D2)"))
 (segment (start 62.325 102.705) (end 62.325 46.389314) (width 0.2) (layer "F.Cu") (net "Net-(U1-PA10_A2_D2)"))
 (segment (start 81.18 43.63) (end 79.47 45.34) (width 0.2) (layer "F.Cu") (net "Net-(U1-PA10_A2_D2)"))
 (segment (start 67.064314 41.65) (end 80.506346 41.65) (width 0.2) (layer "F.Cu") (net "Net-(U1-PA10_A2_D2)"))
 (segment (start 81.18 42.323654) (end 81.18 43.63) (width 0.2) (layer "F.Cu") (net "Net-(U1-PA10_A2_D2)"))
 (segment (start 80.506346 41.65) (end 81.18 42.323654) (width 0.2) (layer "F.Cu") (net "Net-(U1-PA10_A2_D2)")))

